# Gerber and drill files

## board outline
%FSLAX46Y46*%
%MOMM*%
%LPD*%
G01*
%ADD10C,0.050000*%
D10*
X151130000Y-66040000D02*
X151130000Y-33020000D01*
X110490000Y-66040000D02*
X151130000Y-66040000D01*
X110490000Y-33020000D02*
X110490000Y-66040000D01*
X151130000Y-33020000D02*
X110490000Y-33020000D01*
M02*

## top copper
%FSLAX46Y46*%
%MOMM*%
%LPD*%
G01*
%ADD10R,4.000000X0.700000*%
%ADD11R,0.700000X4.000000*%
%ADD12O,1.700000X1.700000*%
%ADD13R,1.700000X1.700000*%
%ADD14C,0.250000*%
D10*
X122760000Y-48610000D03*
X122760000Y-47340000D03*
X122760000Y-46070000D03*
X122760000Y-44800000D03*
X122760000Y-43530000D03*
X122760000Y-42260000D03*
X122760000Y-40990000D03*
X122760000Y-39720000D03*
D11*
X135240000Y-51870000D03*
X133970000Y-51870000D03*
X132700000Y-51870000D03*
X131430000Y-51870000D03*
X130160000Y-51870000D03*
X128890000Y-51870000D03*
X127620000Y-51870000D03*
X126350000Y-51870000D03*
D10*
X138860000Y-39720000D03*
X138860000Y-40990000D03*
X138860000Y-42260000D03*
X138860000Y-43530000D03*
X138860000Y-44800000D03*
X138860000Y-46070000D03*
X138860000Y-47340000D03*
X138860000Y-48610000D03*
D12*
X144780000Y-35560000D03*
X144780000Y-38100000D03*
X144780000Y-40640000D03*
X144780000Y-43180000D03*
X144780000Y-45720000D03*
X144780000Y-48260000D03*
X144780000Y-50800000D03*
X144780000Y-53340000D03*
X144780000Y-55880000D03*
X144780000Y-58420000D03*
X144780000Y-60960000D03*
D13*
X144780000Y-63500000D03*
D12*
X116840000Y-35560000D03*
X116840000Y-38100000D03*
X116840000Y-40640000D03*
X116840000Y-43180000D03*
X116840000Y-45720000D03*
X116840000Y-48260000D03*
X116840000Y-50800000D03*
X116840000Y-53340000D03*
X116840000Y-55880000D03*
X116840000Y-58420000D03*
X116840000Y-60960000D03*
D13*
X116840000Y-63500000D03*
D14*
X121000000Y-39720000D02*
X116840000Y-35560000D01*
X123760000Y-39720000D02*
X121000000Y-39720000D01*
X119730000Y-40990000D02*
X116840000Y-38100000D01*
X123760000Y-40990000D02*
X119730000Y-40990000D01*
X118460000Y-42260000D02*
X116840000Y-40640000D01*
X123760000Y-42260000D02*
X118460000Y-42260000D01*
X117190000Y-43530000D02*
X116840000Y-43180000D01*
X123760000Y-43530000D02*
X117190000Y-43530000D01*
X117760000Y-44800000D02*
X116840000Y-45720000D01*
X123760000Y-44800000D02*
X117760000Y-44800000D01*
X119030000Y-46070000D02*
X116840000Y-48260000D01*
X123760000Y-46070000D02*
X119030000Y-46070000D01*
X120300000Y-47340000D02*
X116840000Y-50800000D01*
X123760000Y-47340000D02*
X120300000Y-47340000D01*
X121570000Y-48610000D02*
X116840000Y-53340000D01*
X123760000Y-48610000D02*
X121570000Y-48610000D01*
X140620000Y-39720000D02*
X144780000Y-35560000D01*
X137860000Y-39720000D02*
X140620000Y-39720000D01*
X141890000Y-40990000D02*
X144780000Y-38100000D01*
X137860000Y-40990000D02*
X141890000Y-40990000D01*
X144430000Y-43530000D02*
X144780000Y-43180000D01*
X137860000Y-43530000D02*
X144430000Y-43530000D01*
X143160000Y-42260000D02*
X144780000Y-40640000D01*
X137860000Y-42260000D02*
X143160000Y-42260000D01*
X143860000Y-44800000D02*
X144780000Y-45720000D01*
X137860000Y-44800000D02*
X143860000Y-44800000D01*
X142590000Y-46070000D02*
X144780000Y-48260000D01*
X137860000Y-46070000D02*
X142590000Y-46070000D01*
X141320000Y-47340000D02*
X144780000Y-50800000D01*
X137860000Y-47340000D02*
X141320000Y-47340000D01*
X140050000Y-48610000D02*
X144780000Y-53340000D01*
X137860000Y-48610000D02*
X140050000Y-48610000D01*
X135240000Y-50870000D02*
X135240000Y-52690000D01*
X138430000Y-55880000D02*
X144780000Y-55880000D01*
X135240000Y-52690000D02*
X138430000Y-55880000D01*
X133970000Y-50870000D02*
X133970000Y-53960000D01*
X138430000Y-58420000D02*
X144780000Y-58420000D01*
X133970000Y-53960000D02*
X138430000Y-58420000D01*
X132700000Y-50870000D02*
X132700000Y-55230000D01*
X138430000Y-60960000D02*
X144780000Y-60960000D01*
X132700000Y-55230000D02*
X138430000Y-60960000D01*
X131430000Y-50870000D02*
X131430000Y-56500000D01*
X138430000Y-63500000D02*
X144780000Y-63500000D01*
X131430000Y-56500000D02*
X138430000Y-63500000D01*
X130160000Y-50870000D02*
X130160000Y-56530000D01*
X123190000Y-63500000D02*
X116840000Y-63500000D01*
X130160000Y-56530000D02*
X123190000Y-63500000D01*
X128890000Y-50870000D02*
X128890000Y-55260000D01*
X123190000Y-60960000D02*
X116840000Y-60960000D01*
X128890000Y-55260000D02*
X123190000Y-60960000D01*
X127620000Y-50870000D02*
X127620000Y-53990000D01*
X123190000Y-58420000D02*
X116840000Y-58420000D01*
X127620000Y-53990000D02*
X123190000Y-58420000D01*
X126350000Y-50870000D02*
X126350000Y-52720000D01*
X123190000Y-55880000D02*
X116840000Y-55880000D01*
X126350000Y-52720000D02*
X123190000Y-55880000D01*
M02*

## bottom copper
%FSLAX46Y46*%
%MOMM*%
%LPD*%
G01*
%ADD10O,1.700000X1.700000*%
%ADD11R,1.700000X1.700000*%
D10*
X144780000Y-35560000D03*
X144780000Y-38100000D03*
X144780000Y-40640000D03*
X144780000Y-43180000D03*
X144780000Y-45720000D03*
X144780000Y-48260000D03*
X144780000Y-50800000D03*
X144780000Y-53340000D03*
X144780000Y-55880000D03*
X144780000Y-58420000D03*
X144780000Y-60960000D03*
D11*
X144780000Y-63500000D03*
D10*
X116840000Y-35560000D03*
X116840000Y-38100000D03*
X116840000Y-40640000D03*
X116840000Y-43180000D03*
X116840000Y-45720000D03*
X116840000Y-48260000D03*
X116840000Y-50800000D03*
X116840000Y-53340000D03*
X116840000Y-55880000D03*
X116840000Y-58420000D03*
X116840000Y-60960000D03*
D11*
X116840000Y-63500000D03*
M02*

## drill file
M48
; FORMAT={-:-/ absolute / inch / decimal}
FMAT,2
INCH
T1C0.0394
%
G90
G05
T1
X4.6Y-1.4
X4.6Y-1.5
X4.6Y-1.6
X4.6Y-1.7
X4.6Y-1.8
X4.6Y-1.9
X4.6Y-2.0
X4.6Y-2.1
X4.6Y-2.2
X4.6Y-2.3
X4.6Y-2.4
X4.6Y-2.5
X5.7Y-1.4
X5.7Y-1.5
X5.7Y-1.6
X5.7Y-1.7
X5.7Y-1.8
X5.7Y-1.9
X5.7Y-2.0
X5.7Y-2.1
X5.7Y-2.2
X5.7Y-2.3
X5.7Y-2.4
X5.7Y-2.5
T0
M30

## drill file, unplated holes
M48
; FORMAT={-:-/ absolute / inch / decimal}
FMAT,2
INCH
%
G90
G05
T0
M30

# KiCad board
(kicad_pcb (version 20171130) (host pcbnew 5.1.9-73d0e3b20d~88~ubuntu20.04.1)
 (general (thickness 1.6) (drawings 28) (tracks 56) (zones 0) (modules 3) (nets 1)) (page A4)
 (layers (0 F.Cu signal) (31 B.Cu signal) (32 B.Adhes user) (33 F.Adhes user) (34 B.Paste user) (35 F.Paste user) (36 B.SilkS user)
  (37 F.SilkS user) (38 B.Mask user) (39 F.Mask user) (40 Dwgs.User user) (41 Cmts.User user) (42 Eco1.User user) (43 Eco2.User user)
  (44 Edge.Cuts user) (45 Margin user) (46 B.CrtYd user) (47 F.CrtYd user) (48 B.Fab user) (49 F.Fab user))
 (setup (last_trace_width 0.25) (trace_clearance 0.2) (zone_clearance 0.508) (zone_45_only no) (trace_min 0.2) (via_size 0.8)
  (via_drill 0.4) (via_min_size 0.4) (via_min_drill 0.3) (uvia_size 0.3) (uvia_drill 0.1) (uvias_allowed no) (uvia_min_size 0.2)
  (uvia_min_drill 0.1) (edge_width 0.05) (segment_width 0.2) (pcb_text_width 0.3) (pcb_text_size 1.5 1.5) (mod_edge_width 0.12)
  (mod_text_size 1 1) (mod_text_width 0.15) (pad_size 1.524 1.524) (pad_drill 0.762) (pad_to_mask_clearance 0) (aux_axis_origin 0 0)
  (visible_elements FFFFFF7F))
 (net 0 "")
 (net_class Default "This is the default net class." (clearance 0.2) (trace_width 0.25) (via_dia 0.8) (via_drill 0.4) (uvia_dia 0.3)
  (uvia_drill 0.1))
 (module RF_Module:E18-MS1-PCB (layer F.Cu) (at 130.81 39.37)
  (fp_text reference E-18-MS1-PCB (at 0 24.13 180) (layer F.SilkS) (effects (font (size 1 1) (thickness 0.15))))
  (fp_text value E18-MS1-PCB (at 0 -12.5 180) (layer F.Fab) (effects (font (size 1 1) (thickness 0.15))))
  (pad 8 smd rect (at -8.05 9.24 270) (size 0.7 4) (layers F.Cu F.Paste F.Mask))
  (pad 7 smd rect (at -8.05 7.97 270) (size 0.7 4) (layers F.Cu F.Paste F.Mask))
  (pad 6 smd rect (at -8.05 6.7 270) (size 0.7 4) (layers F.Cu F.Paste F.Mask))
  (pad 5 smd rect (at -8.05 5.43 270) (size 0.7 4) (layers F.Cu F.Paste F.Mask))
  (pad 4 smd rect (at -8.05 4.16 270) (size 0.7 4) (layers F.Cu F.Paste F.Mask))
  (pad 3 smd rect (at -8.05 2.89 270) (size 0.7 4) (layers F.Cu F.Paste F.Mask))
  (pad 2 smd rect (at -8.05 1.62 270) (size 0.7 4) (layers F.Cu F.Paste F.Mask))
  (pad 1 smd rect (at -8.05 0.35 270) (size 0.7 4) (layers F.Cu F.Paste F.Mask))
  (pad 16 smd rect (at 4.43 12.5 180) (size 0.7 4) (layers F.Cu F.Paste F.Mask))
  (pad 15 smd rect (at 3.16 12.5 180) (size 0.7 4) (layers F.Cu F.Paste F.Mask))
  (pad 14 smd rect (at 1.89 12.5 180) (size 0.7 4) (layers F.Cu F.Paste F.Mask))
  (pad 13 smd rect (at 0.62 12.5 180) (size 0.7 4) (layers F.Cu F.Paste F.Mask))
  (pad 12 smd rect (at -0.65 12.5 180) (size 0.7 4) (layers F.Cu F.Paste F.Mask))
  (pad 11 smd rect (at -1.92 12.5 180) (size 0.7 4) (layers F.Cu F.Paste F.Mask))
  (pad 10 smd rect (at -3.19 12.5 180) (size 0.7 4) (layers F.Cu F.Paste F.Mask))
  (pad 9 smd rect (at -4.46 12.5 180) (size 0.7 4) (layers F.Cu F.Paste F.Mask))
  (pad 24 smd rect (at 8.05 0.35 90) (size 0.7 4) (layers F.Cu F.Paste F.Mask))
  (pad 23 smd rect (at 8.05 1.62 90) (size 0.7 4) (layers F.Cu F.Paste F.Mask))
  (pad 22 smd rect (at 8.05 2.89 90) (size 0.7 4) (layers F.Cu F.Paste F.Mask))
  (pad 21 smd rect (at 8.05 4.16 90) (size 0.7 4) (layers F.Cu F.Paste F.Mask))
  (pad 20 smd rect (at 8.05 5.43 90) (size 0.7 4) (layers F.Cu F.Paste F.Mask))
  (pad 19 smd rect (at 8.05 6.7 90) (size 0.7 4) (layers F.Cu F.Paste F.Mask))
  (pad 18 smd rect (at 8.05 7.97 90) (size 0.7 4) (layers F.Cu F.Paste F.Mask))
  (pad 17 smd rect (at 8.05 9.24 90) (size 0.7 4) (layers F.Cu F.Paste F.Mask)))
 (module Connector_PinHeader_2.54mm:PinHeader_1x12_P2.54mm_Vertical (layer B.Cu) (at 144.78 63.5)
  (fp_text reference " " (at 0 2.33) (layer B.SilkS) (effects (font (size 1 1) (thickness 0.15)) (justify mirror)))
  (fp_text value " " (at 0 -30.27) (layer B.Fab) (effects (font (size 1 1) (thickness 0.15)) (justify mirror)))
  (pad 12 thru_hole oval (at 0 -27.94) (size 1.7 1.7) (drill 1) (layers *.Cu *.Mask))
  (pad 11 thru_hole oval (at 0 -25.4) (size 1.7 1.7) (drill 1) (layers *.Cu *.Mask))
  (pad 10 thru_hole oval (at 0 -22.86) (size 1.7 1.7) (drill 1) (layers *.Cu *.Mask))
  (pad 9 thru_hole oval (at 0 -20.32) (size 1.7 1.7) (drill 1) (layers *.Cu *.Mask))
  (pad 8 thru_hole oval (at 0 -17.78) (size 1.7 1.7) (drill 1) (layers *.Cu *.Mask))
  (pad 7 thru_hole oval (at 0 -15.24) (size 1.7 1.7) (drill 1) (layers *.Cu *.Mask))
  (pad 6 thru_hole oval (at 0 -12.7) (size 1.7 1.7) (drill 1) (layers *.Cu *.Mask))
  (pad 5 thru_hole oval (at 0 -10.16) (size 1.7 1.7) (drill 1) (layers *.Cu *.Mask))
  (pad 4 thru_hole oval (at 0 -7.62) (size 1.7 1.7) (drill 1) (layers *.Cu *.Mask))
  (pad 3 thru_hole oval (at 0 -5.08) (size 1.7 1.7) (drill 1) (layers *.Cu *.Mask))
  (pad 2 thru_hole oval (at 0 -2.54) (size 1.7 1.7) (drill 1) (layers *.Cu *.Mask))
  (pad 1 thru_hole rect (at 0 0) (size 1.7 1.7) (drill 1) (layers *.Cu *.Mask)))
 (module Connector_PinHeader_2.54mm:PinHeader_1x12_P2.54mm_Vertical (layer B.Cu) (at 116.84 63.5)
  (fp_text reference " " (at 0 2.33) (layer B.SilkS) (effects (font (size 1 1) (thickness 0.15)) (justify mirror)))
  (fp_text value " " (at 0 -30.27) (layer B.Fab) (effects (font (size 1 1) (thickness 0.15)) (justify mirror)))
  (pad 12 thru_hole oval (at 0 -27.94) (size 1.7 1.7) (drill 1) (layers *.Cu *.Mask))
  (pad 11 thru_hole oval (at 0 -25.4) (size 1.7 1.7) (drill 1) (layers *.Cu *.Mask))
  (pad 10 thru_hole oval (at 0 -22.86) (size 1.7 1.7) (drill 1) (layers *.Cu *.Mask))
  (pad 9 thru_hole oval (at 0 -20.32) (size 1.7 1.7) (drill 1) (layers *.Cu *.Mask))
  (pad 8 thru_hole oval (at 0 -17.78) (size 1.7 1.7) (drill 1) (layers *.Cu *.Mask))
  (pad 7 thru_hole oval (at 0 -15.24) (size 1.7 1.7) (drill 1) (layers *.Cu *.Mask))
  (pad 6 thru_hole oval (at 0 -12.7) (size 1.7 1.7) (drill 1) (layers *.Cu *.Mask))
  (pad 5 thru_hole oval (at 0 -10.16) (size 1.7 1.7) (drill 1) (layers *.Cu *.Mask))
  (pad 4 thru_hole oval (at 0 -7.62) (size 1.7 1.7) (drill 1) (layers *.Cu *.Mask))
  (pad 3 thru_hole oval (at 0 -5.08) (size 1.7 1.7) (drill 1) (layers *.Cu *.Mask))
  (pad 2 thru_hole oval (at 0 -2.54) (size 1.7 1.7) (drill 1) (layers *.Cu *.Mask))
  (pad 1 thru_hole rect (at 0 0) (size 1.7 1.7) (drill 1) (layers *.Cu *.Mask)))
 (gr_line (start 151.13 66.04) (end 151.13 33.02) (layer Edge.Cuts) (width 0.05))
 (gr_line (start 110.49 66.04) (end 151.13 66.04) (layer Edge.Cuts) (width 0.05))
 (gr_line (start 110.49 33.02) (end 110.49 66.04) (layer Edge.Cuts) (width 0.05))
 (gr_line (start 151.13 33.02) (end 110.49 33.02) (layer Edge.Cuts) (width 0.05))
 (segment (start 121 39.72) (end 116.84 35.56) (width 0.25) (layer F.Cu) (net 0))
 (segment (start 123.76 39.72) (end 121 39.72) (width 0.25) (layer F.Cu) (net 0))
 (segment (start 119.73 40.99) (end 116.84 38.1) (width 0.25) (layer F.Cu) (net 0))
 (segment (start 123.76 40.99) (end 119.73 40.99) (width 0.25) (layer F.Cu) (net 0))
 (segment (start 118.46 42.26) (end 116.84 40.64) (width 0.25) (layer F.Cu) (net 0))
 (segment (start 123.76 42.26) (end 118.46 42.26) (width 0.25) (layer F.Cu) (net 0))
 (segment (start 117.19 43.53) (end 116.84 43.18) (width 0.25) (layer F.Cu) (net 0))
 (segment (start 123.76 43.53) (end 117.19 43.53) (width 0.25) (layer F.Cu) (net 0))
 (segment (start 117.76 44.8) (end 116.84 45.72) (width 0.25) (layer F.Cu) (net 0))
 (segment (start 123.76 44.8) (end 117.76 44.8) (width 0.25) (layer F.Cu) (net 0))
 (segment (start 119.03 46.07) (end 116.84 48.26) (width 0.25) (layer F.Cu) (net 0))
 (segment (start 123.76 46.07) (end 119.03 46.07) (width 0.25) (layer F.Cu) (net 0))
 (segment (start 120.3 47.34) (end 116.84 50.8) (width 0.25) (layer F.Cu) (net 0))
 (segment (start 123.76 47.34) (end 120.3 47.34) (width 0.25) (layer F.Cu) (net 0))
 (segment (start 121.57 48.61) (end 116.84 53.34) (width 0.25) (layer F.Cu) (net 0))
 (segment (start 123.76 48.61) (end 121.57 48.61) (width 0.25) (layer F.Cu) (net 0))
 (segment (start 140.62 39.72) (end 144.78 35.56) (width 0.25) (layer F.Cu) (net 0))
 (segment (start 137.86 39.72) (end 140.62 39.72) (width 0.25) (layer F.Cu) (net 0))
 (segment (start 141.89 40.99) (end 144.78 38.1) (width 0.25) (layer F.Cu) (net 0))
 (segment (start 137.86 40.99) (end 141.89 40.99) (width 0.25) (layer F.Cu) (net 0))
 (segment (start 144.43 43.53) (end 144.78 43.18) (width 0.25) (layer F.Cu) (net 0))
 (segment (start 137.86 43.53) (end 144.43 43.53) (width 0.25) (layer F.Cu) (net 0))
 (segment (start 143.16 42.26) (end 144.78 40.64) (width 0.25) (layer F.Cu) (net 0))
 (segment (start 137.86 42.26) (end 143.16 42.26) (width 0.25) (layer F.Cu) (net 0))
 (segment (start 143.86 44.8) (end 144.78 45.72) (width 0.25) (layer F.Cu) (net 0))
 (segment (start 137.86 44.8) (end 143.86 44.8) (width 0.25) (layer F.Cu) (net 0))
 (segment (start 142.59 46.07) (end 144.78 48.26) (width 0.25) (layer F.Cu) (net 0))
 (segment (start 137.86 46.07) (end 142.59 46.07) (width 0.25) (layer F.Cu) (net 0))
 (segment (start 141.32 47.34) (end 144.78 50.8) (width 0.25) (layer F.Cu) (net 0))
 (segment (start 137.86 47.34) (end 141.32 47.34) (width 0.25) (layer F.Cu) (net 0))
 (segment (start 140.05 48.61) (end 144.78 53.34) (width 0.25) (layer F.Cu) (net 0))
 (segment (start 137.86 48.61) (end 140.05 48.61) (width 0.25) (layer F.Cu) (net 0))
 (segment (start 135.24 50.87) (end 135.24 52.69) (width 0.25) (layer F.Cu) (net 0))
 (segment (start 138.43 55.88) (end 144.78 55.88) (width 0.25) (layer F.Cu) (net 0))
 (segment (start 135.24 52.69) (end 138.43 55.88) (width 0.25) (layer F.Cu) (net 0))
 (segment (start 133.97 50.87) (end 133.97 53.96) (width 0.25) (layer F.Cu) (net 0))
 (segment (start 138.43 58.42) (end 144.78 58.42) (width 0.25) (layer F.Cu) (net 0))
 (segment (start 133.97 53.96) (end 138.43 58.42) (width 0.25) (layer F.Cu) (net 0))
 (segment (start 132.7 50.87) (end 132.7 55.23) (width 0.25) (layer F.Cu) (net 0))
 (segment (start 138.43 60.96) (end 144.78 60.96) (width 0.25) (layer F.Cu) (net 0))
 (segment (start 132.7 55.23) (end 138.43 60.96) (width 0.25) (layer F.Cu) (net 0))
 (segment (start 131.43 50.87) (end 131.43 56.5) (width 0.25) (layer F.Cu) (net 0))
 (segment (start 138.43 63.5) (end 144.78 63.5) (width 0.25) (layer F.Cu) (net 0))
 (segment (start 131.43 56.5) (end 138.43 63.5) (width 0.25) (layer F.Cu) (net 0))
 (segment (start 130.16 50.87) (end 130.16 56.53) (width 0.25) (layer F.Cu) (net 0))
 (segment (start 123.19 63.5) (end 116.84 63.5) (width 0.25) (layer F.Cu) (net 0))
 (segment (start 130.16 56.53) (end 123.19 63.5) (width 0.25) (layer F.Cu) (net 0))
 (segment (start 128.89 50.87) (end 128.89 55.26) (width 0.25) (layer F.Cu) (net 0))
 (segment (start 123.19 60.96) (end 116.84 60.96) (width 0.25) (layer F.Cu) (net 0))
 (segment (start 128.89 55.26) (end 123.19 60.96) (width 0.25) (layer F.Cu) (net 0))
 (segment (start 127.62 50.87) (end 127.62 53.99) (width 0.25) (layer F.Cu) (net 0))
 (segment (start 123.19 58.42) (end 116.84 58.42) (width 0.25) (layer F.Cu) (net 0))
 (segment (start 127.62 53.99) (end 123.19 58.42) (width 0.25) (layer F.Cu) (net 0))
 (segment (start 126.35 50.87) (end 126.35 52.72) (width 0.25) (layer F.Cu) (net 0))
 (segment (start 123.19 55.88) (end 116.84 55.88) (width 0.25) (layer F.Cu) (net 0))
 (segment (start 126.35 52.72) (end 123.19 55.88) (width 0.25) (layer F.Cu) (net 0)))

